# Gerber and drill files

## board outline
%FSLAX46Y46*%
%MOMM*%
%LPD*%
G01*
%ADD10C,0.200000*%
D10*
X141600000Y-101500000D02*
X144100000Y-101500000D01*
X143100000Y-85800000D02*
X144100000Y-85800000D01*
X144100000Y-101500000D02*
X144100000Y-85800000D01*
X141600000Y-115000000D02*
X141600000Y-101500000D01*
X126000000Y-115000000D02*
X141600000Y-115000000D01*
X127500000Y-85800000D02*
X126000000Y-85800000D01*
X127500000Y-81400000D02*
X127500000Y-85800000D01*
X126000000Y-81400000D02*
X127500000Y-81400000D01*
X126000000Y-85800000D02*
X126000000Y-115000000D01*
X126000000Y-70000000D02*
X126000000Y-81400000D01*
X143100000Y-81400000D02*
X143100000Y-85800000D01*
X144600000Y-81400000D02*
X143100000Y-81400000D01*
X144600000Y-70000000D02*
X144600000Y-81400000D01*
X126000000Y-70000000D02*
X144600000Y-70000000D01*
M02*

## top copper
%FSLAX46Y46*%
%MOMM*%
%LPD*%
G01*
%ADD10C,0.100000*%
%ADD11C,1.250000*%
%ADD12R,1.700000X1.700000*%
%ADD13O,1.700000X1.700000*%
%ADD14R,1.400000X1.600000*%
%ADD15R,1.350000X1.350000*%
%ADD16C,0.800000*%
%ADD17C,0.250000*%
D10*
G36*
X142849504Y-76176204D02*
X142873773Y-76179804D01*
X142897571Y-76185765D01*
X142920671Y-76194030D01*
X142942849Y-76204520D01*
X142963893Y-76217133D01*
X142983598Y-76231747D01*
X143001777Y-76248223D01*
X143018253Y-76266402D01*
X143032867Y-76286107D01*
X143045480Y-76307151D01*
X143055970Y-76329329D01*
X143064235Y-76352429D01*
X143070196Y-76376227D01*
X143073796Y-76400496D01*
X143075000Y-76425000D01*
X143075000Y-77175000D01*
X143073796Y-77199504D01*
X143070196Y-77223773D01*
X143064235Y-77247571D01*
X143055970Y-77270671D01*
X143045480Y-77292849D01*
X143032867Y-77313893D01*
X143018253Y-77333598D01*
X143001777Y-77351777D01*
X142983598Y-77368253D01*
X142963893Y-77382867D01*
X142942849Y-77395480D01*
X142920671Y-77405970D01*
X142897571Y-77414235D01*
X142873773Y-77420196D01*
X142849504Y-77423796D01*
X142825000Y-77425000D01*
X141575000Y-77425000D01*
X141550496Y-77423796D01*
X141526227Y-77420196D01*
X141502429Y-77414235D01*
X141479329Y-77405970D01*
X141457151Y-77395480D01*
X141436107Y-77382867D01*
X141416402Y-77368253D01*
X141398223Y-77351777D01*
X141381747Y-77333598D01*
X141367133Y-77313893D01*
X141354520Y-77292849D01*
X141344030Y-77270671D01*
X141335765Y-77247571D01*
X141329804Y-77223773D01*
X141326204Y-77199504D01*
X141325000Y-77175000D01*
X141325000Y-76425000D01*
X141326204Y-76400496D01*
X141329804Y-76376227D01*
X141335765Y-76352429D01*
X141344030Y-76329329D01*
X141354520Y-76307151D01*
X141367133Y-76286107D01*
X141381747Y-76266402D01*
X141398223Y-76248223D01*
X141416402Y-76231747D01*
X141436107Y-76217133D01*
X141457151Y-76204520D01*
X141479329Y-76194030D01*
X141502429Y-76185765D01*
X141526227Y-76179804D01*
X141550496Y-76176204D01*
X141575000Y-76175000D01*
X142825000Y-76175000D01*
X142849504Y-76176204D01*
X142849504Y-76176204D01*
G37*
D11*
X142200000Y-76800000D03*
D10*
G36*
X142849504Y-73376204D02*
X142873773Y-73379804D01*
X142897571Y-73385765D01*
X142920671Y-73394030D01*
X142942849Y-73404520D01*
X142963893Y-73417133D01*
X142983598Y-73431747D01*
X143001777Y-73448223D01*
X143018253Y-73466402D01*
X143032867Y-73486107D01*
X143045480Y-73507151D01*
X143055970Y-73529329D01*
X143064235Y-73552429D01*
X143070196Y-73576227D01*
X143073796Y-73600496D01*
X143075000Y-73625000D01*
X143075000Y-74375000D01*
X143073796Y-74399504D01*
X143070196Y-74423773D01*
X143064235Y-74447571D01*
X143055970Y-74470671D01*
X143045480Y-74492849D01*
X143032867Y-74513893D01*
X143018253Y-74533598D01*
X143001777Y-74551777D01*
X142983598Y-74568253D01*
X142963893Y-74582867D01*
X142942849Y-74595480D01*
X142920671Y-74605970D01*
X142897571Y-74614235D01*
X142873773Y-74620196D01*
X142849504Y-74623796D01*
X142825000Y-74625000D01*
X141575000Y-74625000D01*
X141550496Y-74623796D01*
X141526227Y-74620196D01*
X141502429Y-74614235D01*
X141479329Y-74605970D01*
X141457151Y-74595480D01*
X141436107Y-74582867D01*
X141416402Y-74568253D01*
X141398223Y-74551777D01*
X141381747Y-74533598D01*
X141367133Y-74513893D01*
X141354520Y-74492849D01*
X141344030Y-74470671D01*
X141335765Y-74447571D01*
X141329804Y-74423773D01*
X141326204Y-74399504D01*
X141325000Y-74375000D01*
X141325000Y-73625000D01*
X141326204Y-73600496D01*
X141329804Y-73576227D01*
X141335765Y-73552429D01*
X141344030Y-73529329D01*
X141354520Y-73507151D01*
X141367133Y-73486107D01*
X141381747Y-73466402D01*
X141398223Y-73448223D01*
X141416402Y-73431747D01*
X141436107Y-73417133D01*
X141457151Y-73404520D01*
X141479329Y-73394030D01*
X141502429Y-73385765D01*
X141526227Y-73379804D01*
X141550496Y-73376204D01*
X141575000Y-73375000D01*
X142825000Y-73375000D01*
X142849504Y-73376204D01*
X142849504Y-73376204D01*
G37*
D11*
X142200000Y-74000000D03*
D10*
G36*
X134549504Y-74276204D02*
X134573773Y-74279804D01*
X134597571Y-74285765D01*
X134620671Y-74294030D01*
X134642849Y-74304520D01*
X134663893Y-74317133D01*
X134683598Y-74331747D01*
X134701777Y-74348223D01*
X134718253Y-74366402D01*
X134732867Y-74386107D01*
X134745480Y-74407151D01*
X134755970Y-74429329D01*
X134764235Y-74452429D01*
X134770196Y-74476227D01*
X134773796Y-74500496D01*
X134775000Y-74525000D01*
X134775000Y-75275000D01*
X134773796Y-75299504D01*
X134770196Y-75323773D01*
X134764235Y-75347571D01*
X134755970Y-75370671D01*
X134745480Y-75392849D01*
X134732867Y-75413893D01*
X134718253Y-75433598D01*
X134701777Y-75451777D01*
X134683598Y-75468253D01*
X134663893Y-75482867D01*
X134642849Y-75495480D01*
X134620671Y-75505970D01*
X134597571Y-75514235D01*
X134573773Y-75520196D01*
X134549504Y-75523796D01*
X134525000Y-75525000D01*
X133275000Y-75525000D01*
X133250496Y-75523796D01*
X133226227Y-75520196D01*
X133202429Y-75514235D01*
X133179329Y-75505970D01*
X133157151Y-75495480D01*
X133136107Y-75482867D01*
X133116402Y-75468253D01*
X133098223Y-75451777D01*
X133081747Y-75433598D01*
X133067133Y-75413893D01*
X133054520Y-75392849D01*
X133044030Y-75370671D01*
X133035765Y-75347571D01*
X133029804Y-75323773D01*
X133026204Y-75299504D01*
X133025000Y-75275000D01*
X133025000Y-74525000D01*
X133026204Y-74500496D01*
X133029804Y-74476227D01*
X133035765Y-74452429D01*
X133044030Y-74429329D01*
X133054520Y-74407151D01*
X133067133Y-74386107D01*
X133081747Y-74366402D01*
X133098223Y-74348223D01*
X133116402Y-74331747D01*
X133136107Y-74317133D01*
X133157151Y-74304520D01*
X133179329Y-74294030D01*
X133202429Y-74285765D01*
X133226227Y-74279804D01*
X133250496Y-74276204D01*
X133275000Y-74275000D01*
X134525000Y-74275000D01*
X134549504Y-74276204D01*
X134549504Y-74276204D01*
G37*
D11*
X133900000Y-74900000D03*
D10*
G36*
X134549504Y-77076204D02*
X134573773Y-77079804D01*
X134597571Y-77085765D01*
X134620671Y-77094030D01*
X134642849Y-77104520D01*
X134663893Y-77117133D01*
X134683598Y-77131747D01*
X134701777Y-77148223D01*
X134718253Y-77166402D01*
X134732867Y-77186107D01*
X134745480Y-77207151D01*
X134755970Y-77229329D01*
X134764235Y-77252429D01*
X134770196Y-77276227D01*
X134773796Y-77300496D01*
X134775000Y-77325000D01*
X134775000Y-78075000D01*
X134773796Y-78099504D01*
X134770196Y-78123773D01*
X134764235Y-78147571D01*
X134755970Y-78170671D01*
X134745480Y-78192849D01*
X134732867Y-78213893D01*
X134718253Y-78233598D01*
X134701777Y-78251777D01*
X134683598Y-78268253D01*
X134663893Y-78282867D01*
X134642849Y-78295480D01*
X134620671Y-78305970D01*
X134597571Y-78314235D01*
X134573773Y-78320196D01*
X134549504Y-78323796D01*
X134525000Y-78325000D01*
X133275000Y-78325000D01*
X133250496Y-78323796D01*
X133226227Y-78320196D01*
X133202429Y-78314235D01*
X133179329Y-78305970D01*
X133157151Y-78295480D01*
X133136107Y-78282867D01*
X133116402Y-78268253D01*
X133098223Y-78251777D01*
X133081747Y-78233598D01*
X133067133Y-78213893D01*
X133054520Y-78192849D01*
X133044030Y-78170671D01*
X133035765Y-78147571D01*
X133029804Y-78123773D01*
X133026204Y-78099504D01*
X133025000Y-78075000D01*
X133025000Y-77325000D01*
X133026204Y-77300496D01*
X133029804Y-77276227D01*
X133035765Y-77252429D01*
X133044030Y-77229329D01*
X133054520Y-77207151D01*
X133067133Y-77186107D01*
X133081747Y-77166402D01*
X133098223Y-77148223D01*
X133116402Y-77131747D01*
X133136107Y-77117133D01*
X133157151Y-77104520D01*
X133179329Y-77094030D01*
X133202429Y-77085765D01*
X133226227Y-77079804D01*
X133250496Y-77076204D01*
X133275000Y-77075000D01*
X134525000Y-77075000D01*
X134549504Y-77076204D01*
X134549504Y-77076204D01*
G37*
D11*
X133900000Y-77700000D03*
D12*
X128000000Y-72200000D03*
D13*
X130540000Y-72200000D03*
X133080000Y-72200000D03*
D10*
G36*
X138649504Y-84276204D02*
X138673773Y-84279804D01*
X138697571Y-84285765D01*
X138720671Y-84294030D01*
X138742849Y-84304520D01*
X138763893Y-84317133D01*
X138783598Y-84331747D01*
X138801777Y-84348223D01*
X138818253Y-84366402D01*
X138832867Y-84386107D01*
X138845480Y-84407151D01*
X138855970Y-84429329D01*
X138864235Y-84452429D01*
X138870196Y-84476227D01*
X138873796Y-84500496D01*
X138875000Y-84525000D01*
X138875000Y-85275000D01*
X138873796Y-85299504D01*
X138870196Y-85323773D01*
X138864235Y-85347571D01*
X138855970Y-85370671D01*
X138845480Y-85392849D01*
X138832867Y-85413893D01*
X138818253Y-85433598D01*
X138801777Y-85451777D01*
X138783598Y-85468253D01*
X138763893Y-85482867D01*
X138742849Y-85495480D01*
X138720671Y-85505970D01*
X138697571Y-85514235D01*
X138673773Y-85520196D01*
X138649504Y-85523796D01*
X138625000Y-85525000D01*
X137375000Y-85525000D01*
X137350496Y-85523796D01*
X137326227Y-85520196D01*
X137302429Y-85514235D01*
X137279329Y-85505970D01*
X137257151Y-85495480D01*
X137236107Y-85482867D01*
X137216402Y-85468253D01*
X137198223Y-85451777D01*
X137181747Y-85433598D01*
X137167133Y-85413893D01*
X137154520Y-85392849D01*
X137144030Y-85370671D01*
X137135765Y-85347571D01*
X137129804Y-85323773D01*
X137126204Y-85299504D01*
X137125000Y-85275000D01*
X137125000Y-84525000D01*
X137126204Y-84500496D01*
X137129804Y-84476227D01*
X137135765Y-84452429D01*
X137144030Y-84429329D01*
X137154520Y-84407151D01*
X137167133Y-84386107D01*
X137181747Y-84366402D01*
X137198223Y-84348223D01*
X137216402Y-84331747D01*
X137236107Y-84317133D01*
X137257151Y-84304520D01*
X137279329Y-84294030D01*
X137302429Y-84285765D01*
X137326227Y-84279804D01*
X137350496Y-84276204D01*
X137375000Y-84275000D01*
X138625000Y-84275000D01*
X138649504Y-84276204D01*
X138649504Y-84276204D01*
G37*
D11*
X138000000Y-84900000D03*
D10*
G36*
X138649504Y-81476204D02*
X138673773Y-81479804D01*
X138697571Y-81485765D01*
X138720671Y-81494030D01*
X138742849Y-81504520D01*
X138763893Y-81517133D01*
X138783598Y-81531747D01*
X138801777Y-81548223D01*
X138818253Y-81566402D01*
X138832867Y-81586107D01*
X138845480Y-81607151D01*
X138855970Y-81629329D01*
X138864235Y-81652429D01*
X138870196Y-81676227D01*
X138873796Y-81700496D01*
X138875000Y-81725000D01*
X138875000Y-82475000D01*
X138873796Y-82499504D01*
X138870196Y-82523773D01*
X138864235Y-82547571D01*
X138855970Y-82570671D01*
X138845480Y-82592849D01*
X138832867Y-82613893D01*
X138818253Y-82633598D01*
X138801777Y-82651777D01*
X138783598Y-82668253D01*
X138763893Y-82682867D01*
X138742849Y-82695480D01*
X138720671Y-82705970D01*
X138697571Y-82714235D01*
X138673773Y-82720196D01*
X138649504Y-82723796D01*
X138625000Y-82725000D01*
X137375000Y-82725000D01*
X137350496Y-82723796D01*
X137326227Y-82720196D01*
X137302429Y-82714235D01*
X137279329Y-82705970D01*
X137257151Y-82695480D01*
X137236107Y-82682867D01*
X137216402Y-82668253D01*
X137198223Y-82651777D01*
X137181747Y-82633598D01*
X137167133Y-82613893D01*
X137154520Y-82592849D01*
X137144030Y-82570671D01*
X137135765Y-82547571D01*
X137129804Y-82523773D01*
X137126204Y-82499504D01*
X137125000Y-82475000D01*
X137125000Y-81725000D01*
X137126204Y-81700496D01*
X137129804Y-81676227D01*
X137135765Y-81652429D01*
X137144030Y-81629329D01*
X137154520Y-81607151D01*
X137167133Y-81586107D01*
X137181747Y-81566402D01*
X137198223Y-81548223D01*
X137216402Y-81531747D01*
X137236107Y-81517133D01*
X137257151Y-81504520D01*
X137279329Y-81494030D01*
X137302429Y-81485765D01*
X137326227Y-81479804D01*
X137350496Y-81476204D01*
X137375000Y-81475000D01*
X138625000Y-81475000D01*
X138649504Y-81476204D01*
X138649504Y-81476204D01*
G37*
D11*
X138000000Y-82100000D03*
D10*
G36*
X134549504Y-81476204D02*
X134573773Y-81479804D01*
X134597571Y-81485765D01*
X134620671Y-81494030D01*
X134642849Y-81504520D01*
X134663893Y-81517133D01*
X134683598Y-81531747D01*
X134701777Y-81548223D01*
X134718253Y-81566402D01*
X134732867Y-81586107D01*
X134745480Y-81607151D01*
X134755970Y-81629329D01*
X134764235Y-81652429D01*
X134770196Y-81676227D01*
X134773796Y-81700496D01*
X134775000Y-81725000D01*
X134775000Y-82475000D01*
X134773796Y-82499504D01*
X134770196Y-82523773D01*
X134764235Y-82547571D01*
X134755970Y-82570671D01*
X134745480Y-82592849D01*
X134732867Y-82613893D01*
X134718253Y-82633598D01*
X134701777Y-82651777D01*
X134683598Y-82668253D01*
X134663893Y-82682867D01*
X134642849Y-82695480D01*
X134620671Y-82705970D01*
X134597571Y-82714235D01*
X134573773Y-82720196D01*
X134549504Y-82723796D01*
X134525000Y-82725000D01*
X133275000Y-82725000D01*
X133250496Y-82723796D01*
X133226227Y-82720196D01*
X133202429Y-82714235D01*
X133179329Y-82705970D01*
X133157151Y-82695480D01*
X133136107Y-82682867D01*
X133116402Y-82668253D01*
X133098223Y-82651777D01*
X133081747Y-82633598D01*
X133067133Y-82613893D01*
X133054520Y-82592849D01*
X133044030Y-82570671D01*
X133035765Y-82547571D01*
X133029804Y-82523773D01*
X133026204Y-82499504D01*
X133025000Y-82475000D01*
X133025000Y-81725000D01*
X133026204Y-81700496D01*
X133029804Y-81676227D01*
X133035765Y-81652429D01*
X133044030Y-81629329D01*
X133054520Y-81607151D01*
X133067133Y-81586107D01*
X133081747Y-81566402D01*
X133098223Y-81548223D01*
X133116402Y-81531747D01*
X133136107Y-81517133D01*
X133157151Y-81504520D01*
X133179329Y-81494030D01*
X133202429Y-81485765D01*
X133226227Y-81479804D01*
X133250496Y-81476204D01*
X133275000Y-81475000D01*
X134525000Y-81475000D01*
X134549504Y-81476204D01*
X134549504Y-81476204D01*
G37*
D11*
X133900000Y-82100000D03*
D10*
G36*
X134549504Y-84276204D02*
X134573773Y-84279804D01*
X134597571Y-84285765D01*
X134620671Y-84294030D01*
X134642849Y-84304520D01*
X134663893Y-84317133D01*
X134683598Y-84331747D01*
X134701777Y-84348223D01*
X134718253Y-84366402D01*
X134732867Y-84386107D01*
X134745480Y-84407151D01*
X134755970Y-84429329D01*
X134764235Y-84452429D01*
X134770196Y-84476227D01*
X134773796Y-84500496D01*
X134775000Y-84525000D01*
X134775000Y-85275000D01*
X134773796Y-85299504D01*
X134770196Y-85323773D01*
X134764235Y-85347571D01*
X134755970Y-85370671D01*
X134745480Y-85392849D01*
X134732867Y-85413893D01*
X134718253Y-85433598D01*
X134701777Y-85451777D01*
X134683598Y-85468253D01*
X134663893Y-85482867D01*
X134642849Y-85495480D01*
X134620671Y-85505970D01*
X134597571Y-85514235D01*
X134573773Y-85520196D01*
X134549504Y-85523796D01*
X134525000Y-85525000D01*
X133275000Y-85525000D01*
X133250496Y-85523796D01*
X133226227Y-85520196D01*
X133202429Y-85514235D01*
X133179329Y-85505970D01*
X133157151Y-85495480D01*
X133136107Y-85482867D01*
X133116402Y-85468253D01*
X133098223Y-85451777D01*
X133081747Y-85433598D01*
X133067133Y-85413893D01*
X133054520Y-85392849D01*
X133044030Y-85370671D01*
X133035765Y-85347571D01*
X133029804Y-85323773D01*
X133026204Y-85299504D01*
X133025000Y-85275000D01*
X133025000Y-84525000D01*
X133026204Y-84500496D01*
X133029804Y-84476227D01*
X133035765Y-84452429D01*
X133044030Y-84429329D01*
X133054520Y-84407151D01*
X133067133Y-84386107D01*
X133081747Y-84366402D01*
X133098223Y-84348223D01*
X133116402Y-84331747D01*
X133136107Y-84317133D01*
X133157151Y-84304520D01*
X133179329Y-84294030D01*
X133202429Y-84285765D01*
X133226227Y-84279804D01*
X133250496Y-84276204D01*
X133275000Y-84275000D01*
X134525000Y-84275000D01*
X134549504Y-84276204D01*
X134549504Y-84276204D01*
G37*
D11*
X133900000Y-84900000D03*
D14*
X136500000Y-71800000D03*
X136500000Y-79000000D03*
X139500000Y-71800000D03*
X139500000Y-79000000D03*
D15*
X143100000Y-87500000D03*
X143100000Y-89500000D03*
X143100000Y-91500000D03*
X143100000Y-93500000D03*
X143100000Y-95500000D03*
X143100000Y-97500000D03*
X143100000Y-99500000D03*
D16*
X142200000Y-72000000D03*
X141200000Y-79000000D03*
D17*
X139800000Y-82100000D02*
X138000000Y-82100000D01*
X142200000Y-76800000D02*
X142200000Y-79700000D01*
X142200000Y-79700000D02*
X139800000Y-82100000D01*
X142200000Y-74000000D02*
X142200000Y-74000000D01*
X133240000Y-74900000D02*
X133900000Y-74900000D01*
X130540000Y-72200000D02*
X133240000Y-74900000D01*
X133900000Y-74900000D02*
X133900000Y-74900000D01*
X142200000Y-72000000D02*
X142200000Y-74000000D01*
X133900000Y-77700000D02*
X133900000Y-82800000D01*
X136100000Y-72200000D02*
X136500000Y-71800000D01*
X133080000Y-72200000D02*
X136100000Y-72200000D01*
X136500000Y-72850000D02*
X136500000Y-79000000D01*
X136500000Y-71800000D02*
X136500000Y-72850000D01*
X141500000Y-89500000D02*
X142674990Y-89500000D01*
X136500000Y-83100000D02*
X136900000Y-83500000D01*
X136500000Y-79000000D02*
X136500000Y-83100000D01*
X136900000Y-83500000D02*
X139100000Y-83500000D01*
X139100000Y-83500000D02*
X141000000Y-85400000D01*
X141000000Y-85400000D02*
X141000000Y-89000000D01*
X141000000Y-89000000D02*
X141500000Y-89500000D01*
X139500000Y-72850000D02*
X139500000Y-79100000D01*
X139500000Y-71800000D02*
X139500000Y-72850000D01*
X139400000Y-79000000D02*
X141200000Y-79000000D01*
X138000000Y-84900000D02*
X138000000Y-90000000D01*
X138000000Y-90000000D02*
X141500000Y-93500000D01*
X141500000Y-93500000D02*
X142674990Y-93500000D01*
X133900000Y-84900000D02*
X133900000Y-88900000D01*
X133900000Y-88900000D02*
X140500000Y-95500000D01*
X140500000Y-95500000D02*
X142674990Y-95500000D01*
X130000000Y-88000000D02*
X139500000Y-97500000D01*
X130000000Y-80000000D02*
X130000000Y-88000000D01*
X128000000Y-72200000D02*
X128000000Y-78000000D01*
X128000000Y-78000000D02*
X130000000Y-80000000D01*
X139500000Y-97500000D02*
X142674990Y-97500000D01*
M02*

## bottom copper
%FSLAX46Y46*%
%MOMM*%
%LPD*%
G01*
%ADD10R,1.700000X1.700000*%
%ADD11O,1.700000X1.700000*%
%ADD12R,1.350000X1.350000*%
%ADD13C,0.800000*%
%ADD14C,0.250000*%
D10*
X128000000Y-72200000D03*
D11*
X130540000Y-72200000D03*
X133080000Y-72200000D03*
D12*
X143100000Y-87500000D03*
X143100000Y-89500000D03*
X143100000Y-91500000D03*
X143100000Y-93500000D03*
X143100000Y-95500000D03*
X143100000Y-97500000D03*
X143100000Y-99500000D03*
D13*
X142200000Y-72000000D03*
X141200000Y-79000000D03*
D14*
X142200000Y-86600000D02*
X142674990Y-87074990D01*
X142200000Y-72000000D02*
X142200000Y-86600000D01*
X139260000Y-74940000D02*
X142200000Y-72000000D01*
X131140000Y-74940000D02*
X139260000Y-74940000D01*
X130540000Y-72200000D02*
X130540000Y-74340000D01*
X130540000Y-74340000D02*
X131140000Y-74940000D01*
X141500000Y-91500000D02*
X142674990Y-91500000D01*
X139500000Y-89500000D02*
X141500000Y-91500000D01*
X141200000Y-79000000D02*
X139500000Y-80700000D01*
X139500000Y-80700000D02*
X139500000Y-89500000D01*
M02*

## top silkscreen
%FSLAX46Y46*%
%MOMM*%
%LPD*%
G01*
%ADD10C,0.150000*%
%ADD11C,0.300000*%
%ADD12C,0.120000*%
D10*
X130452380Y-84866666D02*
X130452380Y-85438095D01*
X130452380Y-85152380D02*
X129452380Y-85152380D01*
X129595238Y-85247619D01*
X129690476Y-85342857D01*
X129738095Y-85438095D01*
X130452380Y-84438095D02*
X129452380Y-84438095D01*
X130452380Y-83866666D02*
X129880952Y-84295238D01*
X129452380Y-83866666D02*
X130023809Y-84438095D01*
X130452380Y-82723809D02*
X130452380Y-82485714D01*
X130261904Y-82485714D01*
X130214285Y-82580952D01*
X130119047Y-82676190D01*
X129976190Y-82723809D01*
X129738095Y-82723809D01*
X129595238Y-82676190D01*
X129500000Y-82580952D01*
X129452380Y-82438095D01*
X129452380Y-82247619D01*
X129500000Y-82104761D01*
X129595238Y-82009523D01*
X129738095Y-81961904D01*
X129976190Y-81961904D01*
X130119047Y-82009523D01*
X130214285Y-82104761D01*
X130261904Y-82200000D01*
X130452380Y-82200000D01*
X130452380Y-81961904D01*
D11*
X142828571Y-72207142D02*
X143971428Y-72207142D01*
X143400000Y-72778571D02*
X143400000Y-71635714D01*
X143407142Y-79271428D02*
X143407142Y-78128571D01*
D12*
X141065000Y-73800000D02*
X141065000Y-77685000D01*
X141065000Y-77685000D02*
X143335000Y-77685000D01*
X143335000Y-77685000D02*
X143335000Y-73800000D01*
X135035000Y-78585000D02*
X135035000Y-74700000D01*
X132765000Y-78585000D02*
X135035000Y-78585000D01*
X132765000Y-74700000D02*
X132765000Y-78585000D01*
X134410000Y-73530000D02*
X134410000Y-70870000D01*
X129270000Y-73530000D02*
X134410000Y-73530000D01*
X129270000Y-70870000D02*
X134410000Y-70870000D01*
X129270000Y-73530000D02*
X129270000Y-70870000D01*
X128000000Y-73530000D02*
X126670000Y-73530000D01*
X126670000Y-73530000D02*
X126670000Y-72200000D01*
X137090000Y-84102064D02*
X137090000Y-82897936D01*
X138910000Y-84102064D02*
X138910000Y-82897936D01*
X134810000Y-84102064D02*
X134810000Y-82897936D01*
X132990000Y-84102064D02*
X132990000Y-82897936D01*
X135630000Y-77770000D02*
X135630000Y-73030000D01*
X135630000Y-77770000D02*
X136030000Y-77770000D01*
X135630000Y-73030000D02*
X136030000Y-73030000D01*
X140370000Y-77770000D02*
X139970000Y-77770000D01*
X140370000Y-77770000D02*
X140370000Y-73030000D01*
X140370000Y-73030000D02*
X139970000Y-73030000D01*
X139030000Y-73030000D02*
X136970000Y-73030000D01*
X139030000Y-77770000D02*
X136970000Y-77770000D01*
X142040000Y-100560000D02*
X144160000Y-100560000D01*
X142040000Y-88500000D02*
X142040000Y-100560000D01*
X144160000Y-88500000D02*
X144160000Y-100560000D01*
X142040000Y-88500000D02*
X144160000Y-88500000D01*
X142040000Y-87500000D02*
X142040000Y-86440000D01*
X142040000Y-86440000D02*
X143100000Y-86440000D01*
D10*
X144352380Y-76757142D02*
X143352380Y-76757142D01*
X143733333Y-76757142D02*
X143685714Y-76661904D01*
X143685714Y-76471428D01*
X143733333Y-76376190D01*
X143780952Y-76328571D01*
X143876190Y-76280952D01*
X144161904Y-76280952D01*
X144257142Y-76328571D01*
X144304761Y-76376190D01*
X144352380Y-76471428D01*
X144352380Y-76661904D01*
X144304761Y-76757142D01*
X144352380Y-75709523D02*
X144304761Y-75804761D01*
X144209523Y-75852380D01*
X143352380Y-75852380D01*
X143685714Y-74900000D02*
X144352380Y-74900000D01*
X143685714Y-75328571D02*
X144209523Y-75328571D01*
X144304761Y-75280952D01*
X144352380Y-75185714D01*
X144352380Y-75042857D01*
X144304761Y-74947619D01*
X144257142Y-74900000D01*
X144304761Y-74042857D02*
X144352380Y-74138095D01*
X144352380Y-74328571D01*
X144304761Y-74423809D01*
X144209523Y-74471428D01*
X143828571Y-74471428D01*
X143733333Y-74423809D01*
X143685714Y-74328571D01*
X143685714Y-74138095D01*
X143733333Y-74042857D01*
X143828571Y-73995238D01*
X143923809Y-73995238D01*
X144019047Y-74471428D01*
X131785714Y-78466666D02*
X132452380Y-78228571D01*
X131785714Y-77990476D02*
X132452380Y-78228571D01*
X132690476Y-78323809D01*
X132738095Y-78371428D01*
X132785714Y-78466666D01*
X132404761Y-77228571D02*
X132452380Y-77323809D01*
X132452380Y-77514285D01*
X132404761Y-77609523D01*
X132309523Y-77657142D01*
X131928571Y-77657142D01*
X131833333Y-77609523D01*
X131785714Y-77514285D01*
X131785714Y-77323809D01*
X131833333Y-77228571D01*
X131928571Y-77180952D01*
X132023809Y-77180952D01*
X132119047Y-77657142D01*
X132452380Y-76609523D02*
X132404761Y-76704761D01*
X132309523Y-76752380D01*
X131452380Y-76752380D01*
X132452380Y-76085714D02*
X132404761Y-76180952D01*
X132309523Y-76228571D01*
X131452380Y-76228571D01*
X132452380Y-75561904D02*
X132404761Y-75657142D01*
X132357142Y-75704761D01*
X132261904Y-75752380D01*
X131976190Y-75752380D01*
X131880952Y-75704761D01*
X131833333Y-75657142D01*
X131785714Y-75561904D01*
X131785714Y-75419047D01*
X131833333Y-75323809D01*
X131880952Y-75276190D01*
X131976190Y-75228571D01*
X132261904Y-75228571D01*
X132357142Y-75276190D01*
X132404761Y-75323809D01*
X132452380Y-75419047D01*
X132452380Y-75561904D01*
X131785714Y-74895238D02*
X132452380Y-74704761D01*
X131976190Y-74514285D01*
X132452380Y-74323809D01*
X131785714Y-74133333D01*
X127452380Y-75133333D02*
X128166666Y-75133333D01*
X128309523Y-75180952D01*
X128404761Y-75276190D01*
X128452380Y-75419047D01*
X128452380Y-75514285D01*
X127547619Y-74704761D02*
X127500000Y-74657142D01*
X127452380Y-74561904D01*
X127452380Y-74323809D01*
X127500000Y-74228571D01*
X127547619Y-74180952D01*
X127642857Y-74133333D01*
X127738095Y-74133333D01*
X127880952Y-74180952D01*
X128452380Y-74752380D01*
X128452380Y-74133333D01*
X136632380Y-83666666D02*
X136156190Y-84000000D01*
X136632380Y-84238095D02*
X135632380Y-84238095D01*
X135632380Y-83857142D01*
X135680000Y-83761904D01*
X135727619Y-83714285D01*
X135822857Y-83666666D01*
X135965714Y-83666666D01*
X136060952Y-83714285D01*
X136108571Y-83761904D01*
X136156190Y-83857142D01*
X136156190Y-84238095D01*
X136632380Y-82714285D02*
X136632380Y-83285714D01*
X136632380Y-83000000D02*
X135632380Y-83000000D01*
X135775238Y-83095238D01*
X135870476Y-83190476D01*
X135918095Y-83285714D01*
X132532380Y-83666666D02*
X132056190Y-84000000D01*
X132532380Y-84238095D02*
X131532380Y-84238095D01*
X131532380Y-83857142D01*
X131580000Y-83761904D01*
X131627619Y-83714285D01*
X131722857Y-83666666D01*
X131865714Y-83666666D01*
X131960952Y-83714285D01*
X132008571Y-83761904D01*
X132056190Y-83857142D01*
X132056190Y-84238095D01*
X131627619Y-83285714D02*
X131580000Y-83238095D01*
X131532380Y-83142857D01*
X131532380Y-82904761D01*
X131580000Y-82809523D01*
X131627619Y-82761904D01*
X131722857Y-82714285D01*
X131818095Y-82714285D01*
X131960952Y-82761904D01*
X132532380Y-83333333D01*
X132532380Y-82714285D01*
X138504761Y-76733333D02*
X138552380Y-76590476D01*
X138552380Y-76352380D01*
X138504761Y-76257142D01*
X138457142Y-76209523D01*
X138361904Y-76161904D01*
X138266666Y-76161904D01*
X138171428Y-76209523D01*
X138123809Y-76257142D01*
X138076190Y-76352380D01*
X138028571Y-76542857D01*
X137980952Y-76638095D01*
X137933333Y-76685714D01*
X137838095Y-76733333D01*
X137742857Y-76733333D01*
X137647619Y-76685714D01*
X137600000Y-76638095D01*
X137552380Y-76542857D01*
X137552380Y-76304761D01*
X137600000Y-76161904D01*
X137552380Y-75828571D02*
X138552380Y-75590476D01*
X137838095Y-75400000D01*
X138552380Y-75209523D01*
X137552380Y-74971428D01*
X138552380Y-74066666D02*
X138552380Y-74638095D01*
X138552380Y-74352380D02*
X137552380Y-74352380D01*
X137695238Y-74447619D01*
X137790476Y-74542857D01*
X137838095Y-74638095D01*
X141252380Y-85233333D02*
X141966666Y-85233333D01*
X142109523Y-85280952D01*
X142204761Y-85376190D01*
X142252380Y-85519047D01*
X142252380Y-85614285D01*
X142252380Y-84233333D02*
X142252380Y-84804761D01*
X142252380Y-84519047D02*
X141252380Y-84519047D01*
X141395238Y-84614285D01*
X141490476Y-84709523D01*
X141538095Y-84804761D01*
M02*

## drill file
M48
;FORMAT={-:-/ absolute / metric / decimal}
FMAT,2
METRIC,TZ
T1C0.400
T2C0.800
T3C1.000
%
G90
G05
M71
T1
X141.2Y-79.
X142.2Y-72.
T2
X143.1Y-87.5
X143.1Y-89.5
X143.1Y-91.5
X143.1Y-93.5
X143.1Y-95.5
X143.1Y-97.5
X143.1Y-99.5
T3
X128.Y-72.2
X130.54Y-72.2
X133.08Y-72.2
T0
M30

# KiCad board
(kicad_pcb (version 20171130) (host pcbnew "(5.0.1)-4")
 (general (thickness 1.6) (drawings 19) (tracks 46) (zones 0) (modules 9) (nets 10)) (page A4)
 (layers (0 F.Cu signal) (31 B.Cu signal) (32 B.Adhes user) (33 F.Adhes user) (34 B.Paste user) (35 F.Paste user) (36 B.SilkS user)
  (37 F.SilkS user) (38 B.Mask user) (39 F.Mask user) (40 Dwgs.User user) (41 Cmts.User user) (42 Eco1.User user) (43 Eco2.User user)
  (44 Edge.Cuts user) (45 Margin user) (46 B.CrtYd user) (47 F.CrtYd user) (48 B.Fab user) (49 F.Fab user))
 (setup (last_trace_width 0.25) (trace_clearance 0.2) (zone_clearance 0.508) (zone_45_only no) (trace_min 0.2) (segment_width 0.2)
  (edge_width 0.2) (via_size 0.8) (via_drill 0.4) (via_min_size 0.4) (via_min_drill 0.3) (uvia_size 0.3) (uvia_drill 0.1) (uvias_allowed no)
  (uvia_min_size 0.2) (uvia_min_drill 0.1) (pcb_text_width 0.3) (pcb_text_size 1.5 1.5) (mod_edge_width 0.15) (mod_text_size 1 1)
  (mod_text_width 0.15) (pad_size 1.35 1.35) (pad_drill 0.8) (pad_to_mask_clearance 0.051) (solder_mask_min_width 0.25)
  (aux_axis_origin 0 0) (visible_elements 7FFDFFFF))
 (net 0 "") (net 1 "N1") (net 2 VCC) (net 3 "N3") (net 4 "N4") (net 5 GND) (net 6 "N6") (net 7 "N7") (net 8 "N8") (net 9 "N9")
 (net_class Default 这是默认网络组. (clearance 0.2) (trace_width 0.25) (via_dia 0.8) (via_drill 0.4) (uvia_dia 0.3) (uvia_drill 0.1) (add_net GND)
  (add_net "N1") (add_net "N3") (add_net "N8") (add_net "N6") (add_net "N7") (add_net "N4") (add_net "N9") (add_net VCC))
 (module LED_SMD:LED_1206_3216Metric (layer F.Cu) (at 142.2 75.4 90)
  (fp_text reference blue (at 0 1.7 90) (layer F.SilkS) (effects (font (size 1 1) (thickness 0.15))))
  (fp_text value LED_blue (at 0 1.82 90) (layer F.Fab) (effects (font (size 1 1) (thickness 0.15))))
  (fp_line (start 1.6 -1.135) (end -2.285 -1.135) (layer F.SilkS) (width 0.12))
  (fp_line (start -2.285 -1.135) (end -2.285 1.135) (layer F.SilkS) (width 0.12))
  (fp_line (start -2.285 1.135) (end 1.6 1.135) (layer F.SilkS) (width 0.12))
  (pad 1 smd roundrect (at -1.4 0 90) (size 1.25 1.75) (layers F.Cu F.Paste F.Mask) (roundrect_rratio 0.2) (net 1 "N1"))
  (pad 2 smd roundrect (at 1.4 0 90) (size 1.25 1.75) (layers F.Cu F.Paste F.Mask) (roundrect_rratio 0.2) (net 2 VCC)))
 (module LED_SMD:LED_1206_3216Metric (layer F.Cu) (at 133.9 76.3 90)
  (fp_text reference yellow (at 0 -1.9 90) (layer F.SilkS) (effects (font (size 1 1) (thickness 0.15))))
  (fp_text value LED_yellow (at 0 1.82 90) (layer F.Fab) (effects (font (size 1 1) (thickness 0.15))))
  (fp_line (start -2.285 1.135) (end 1.6 1.135) (layer F.SilkS) (width 0.12))
  (fp_line (start -2.285 -1.135) (end -2.285 1.135) (layer F.SilkS) (width 0.12))
  (fp_line (start 1.6 -1.135) (end -2.285 -1.135) (layer F.SilkS) (width 0.12))
  (pad 2 smd roundrect (at 1.4 0 90) (size 1.25 1.75) (layers F.Cu F.Paste F.Mask) (roundrect_rratio 0.2) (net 2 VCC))
  (pad 1 smd roundrect (at -1.4 0 90) (size 1.25 1.75) (layers F.Cu F.Paste F.Mask) (roundrect_rratio 0.2) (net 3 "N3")))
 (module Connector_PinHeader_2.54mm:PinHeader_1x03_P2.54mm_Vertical (layer F.Cu) (at 128 72.2 90)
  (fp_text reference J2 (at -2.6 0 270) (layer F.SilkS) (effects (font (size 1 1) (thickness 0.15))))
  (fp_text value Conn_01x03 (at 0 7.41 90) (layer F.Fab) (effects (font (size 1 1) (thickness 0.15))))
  (fp_line (start -1.33 6.41) (end 1.33 6.41) (layer F.SilkS) (width 0.12))
  (fp_line (start -1.33 1.27) (end -1.33 6.41) (layer F.SilkS) (width 0.12))
  (fp_line (start 1.33 1.27) (end 1.33 6.41) (layer F.SilkS) (width 0.12))
  (fp_line (start -1.33 1.27) (end 1.33 1.27) (layer F.SilkS) (width 0.12))
  (fp_line (start -1.33 0) (end -1.33 -1.33) (layer F.SilkS) (width 0.12))
  (fp_line (start -1.33 -1.33) (end 0 -1.33) (layer F.SilkS) (width 0.12))
  (pad 1 thru_hole rect (at 0 0 90) (size 1.7 1.7) (drill 1) (layers *.Cu *.Mask) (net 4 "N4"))
  (pad 2 thru_hole oval (at 0 2.54 90) (size 1.7 1.7) (drill 1) (layers *.Cu *.Mask) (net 2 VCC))
  (pad 3 thru_hole oval (at 0 5.08 90) (size 1.7 1.7) (drill 1) (layers *.Cu *.Mask) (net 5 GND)))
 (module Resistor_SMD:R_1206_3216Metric (layer F.Cu) (at 138 83.5 90)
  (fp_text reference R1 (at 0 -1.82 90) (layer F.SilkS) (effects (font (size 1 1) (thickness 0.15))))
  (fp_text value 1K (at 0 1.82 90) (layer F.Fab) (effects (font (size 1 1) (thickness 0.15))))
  (fp_line (start -0.602064 -0.91) (end 0.602064 -0.91) (layer F.SilkS) (width 0.12))
  (fp_line (start -0.602064 0.91) (end 0.602064 0.91) (layer F.SilkS) (width 0.12))
  (pad 1 smd roundrect (at -1.4 0 90) (size 1.25 1.75) (layers F.Cu F.Paste F.Mask) (roundrect_rratio 0.2) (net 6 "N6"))
  (pad 2 smd roundrect (at 1.4 0 90) (size 1.25 1.75) (layers F.Cu F.Paste F.Mask) (roundrect_rratio 0.2) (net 1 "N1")))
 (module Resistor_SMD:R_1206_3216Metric (layer F.Cu) (at 133.9 83.5 90)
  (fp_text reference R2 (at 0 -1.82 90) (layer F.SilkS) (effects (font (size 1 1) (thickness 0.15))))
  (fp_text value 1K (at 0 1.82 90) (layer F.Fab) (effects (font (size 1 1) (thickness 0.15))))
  (fp_line (start -0.602064 0.91) (end 0.602064 0.91) (layer F.SilkS) (width 0.12))
  (fp_line (start -0.602064 -0.91) (end 0.602064 -0.91) (layer F.SilkS) (width 0.12))
  (pad 2 smd roundrect (at 1.4 0 90) (size 1.25 1.75) (layers F.Cu F.Paste F.Mask) (roundrect_rratio 0.2) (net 3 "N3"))
  (pad 1 smd roundrect (at -1.4 0 90) (size 1.25 1.75) (layers F.Cu F.Paste F.Mask) (roundrect_rratio 0.2) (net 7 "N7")))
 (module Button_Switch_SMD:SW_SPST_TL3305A (layer F.Cu) (at 138 75.4 90)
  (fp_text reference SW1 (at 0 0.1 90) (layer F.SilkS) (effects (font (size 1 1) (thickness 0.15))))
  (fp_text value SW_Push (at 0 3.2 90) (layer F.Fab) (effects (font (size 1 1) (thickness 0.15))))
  (fp_line (start -2.37 -2.37) (end 2.37 -2.37) (layer F.SilkS) (width 0.12))
  (fp_line (start -2.37 -2.37) (end -2.37 -1.97) (layer F.SilkS) (width 0.12))
  (fp_line (start 2.37 -2.37) (end 2.37 -1.97) (layer F.SilkS) (width 0.12))
  (fp_line (start -2.37 2.37) (end -2.37 1.97) (layer F.SilkS) (width 0.12))
  (fp_line (start -2.37 2.37) (end 2.37 2.37) (layer F.SilkS) (width 0.12))
  (fp_line (start 2.37 2.37) (end 2.37 1.97) (layer F.SilkS) (width 0.12))
  (fp_line (start 2.37 1.03) (end 2.37 -1.03) (layer F.SilkS) (width 0.12))
  (fp_line (start -2.37 1.03) (end -2.37 -1.03) (layer F.SilkS) (width 0.12))
  (pad 1 smd rect (at 3.6 -1.5 90) (size 1.6 1.4) (layers F.Cu F.Paste F.Mask) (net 5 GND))
  (pad 1 smd rect (at -3.6 -1.5 90) (size 1.6 1.4) (layers F.Cu F.Paste F.Mask) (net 5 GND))
  (pad 2 smd rect (at 3.6 1.5 90) (size 1.6 1.4) (layers F.Cu F.Paste F.Mask) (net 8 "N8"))
  (pad 2 smd rect (at -3.6 1.5 90) (size 1.6 1.4) (layers F.Cu F.Paste F.Mask) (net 8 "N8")))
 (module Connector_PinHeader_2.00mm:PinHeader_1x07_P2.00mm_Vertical (layer F.Cu) (at 143.1 87.5)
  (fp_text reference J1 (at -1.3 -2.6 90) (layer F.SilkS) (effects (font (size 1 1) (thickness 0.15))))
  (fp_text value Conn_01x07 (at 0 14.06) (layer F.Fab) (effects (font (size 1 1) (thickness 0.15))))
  (fp_line (start -1.06 13.06) (end 1.06 13.06) (layer F.SilkS) (width 0.12))
  (fp_line (start -1.06 1) (end -1.06 13.06) (layer F.SilkS) (width 0.12))
  (fp_line (start 1.06 1) (end 1.06 13.06) (layer F.SilkS) (width 0.12))
  (fp_line (start -1.06 1) (end 1.06 1) (layer F.SilkS) (width 0.12))
  (fp_line (start -1.06 0) (end -1.06 -1.06) (layer F.SilkS) (width 0.12))
  (fp_line (start -1.06 -1.06) (end 0 -1.06) (layer F.SilkS) (width 0.12))
  (pad 1 thru_hole rect (at 0 0) (size 1.35 1.35) (drill 0.8) (layers *.Cu *.Mask) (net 2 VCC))
  (pad 2 thru_hole rect (at 0 2) (size 1.35 1.35) (drill 0.8) (layers *.Cu *.Mask) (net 5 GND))
  (pad 3 thru_hole rect (at 0 4) (size 1.35 1.35) (drill 0.8) (layers *.Cu *.Mask) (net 8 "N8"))
  (pad 4 thru_hole rect (at 0 6) (size 1.35 1.35) (drill 0.8) (layers *.Cu *.Mask) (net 6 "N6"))
  (pad 5 thru_hole rect (at 0 8) (size 1.35 1.35) (drill 0.8) (layers *.Cu *.Mask) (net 7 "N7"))
  (pad 6 thru_hole rect (at 0 10) (size 1.35 1.35) (drill 0.8) (layers *.Cu *.Mask) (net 4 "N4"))
  (pad 7 thru_hole rect (at 0 12) (size 1.35 1.35) (drill 0.8) (layers *.Cu *.Mask) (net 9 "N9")))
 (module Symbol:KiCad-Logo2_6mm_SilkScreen (layer B.Cu) (at 134 110)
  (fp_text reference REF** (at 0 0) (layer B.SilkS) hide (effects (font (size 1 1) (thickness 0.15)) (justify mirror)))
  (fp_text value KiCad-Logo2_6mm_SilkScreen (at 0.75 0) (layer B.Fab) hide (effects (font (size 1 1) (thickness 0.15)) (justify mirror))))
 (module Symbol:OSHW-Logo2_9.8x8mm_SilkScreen (layer B.Cu) (at 134 100.8)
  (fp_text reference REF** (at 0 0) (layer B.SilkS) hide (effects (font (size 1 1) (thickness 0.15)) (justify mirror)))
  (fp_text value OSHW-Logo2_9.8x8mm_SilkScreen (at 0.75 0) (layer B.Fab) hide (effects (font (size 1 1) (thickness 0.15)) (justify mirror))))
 (gr_line (start 141.6 101.5) (end 144.1 101.5) (layer Edge.Cuts) (width 0.2))
 (gr_line (start 143.1 85.8) (end 144.1 85.8) (layer Edge.Cuts) (width 0.2))
 (gr_line (start 144.1 101.5) (end 144.1 85.8) (layer Edge.Cuts) (width 0.2))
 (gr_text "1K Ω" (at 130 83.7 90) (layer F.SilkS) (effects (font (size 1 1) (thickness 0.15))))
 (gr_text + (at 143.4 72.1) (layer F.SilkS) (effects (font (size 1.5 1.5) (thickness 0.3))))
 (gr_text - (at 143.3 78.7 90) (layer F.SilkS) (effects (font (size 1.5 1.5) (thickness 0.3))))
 (gr_line (start 141.6 115) (end 141.6 101.5) (layer Edge.Cuts) (width 0.2))
 (gr_line (start 126 115) (end 141.6 115) (layer Edge.Cuts) (width 0.2))
 (gr_line (start 127.5 85.8) (end 126 85.8) (layer Edge.Cuts) (width 0.2))
 (gr_line (start 127.5 81.4) (end 127.5 85.8) (layer Edge.Cuts) (width 0.2))
 (gr_line (start 126 81.4) (end 127.5 81.4) (layer Edge.Cuts) (width 0.2))
 (gr_line (start 126 85.8) (end 126 115) (layer Edge.Cuts) (width 0.2))
 (gr_line (start 126 70) (end 126 81.4) (layer Edge.Cuts) (width 0.2))
 (gr_line (start 143.1 81.4) (end 143.1 85.8) (layer Edge.Cuts) (width 0.2))
 (gr_line (start 144.6 81.4) (end 143.1 81.4) (layer Edge.Cuts) (width 0.2))
 (gr_line (start 144.6 70) (end 144.6 81.4) (layer Edge.Cuts) (width 0.2))
 (gr_line (start 126 70) (end 144.6 70) (layer Edge.Cuts) (width 0.2))
 (segment (start 139.8 82.1) (end 138 82.1) (width 0.25) (layer F.Cu) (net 1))
 (segment (start 142.2 76.8) (end 142.2 79.7) (width 0.25) (layer F.Cu) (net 1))
 (segment (start 142.2 79.7) (end 139.8 82.1) (width 0.25) (layer F.Cu) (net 1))
 (segment (start 142.2 74) (end 142.2 74) (width 0.25) (layer F.Cu) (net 2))
 (segment (start 133.24 74.9) (end 133.9 74.9) (width 0.25) (layer F.Cu) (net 2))
 (segment (start 130.54 72.2) (end 133.24 74.9) (width 0.25) (layer F.Cu) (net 2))
 (segment (start 133.9 74.9) (end 133.9 74.9) (width 0.25) (layer F.Cu) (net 2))
 (via (at 142.2 72) (size 0.8) (drill 0.4) (layers F.Cu B.Cu) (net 2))
 (segment (start 142.2 72) (end 142.2 74) (width 0.25) (layer F.Cu) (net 2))
 (segment (start 142.2 86.6) (end 142.67499 87.07499) (width 0.25) (layer B.Cu) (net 2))
 (segment (start 142.2 72) (end 142.2 86.6) (width 0.25) (layer B.Cu) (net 2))
 (segment (start 139.26 74.94) (end 142.2 72) (width 0.25) (layer B.Cu) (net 2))
 (segment (start 131.14 74.94) (end 139.26 74.94) (width 0.25) (layer B.Cu) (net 2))
 (segment (start 130.54 72.2) (end 130.54 74.34) (width 0.25) (layer B.Cu) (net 2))
 (segment (start 130.54 74.34) (end 131.14 74.94) (width 0.25) (layer B.Cu) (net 2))
 (segment (start 133.9 77.7) (end 133.9 82.8) (width 0.25) (layer F.Cu) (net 3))
 (segment (start 136.1 72.2) (end 136.5 71.8) (width 0.25) (layer F.Cu) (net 5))
 (segment (start 133.08 72.2) (end 136.1 72.2) (width 0.25) (layer F.Cu) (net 5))
 (segment (start 136.5 72.85) (end 136.5 79) (width 0.25) (layer F.Cu) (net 5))
 (segment (start 136.5 71.8) (end 136.5 72.85) (width 0.25) (layer F.Cu) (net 5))
 (segment (start 141.5 89.5) (end 142.67499 89.5) (width 0.25) (layer F.Cu) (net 5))
 (segment (start 136.5 83.1) (end 136.9 83.5) (width 0.25) (layer F.Cu) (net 5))
 (segment (start 136.5 79) (end 136.5 83.1) (width 0.25) (layer F.Cu) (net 5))
 (segment (start 136.9 83.5) (end 139.1 83.5) (width 0.25) (layer F.Cu) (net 5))
 (segment (start 139.1 83.5) (end 141 85.4) (width 0.25) (layer F.Cu) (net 5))
 (segment (start 141 85.4) (end 141 89) (width 0.25) (layer F.Cu) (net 5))
 (segment (start 141 89) (end 141.5 89.5) (width 0.25) (layer F.Cu) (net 5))
 (via (at 141.2 79) (size 0.8) (drill 0.4) (layers F.Cu B.Cu) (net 8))
 (segment (start 139.5 72.85) (end 139.5 79.1) (width 0.25) (layer F.Cu) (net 8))
 (segment (start 139.5 71.8) (end 139.5 72.85) (width 0.25) (layer F.Cu) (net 8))
 (segment (start 139.4 79) (end 141.2 79) (width 0.25) (layer F.Cu) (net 8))
 (segment (start 141.5 91.5) (end 142.67499 91.5) (width 0.25) (layer B.Cu) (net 8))
 (segment (start 139.5 89.5) (end 141.5 91.5) (width 0.25) (layer B.Cu) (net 8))
 (segment (start 141.2 79) (end 139.5 80.7) (width 0.25) (layer B.Cu) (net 8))
 (segment (start 139.5 80.7) (end 139.5 89.5) (width 0.25) (layer B.Cu) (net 8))
 (segment (start 138 84.9) (end 138 90) (width 0.25) (layer F.Cu) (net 6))
 (segment (start 138 90) (end 141.5 93.5) (width 0.25) (layer F.Cu) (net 6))
 (segment (start 141.5 93.5) (end 142.67499 93.5) (width 0.25) (layer F.Cu) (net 6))
 (segment (start 133.9 84.9) (end 133.9 88.9) (width 0.25) (layer F.Cu) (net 7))
 (segment (start 133.9 88.9) (end 140.5 95.5) (width 0.25) (layer F.Cu) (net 7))
 (segment (start 140.5 95.5) (end 142.67499 95.5) (width 0.25) (layer F.Cu) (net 7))
 (segment (start 130 88) (end 139.5 97.5) (width 0.25) (layer F.Cu) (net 4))
 (segment (start 130 80) (end 130 88) (width 0.25) (layer F.Cu) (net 4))
 (segment (start 128 72.2) (end 128 78) (width 0.25) (layer F.Cu) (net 4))
 (segment (start 128 78) (end 130 80) (width 0.25) (layer F.Cu) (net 4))
 (segment (start 139.5 97.5) (end 142.67499 97.5) (width 0.25) (layer F.Cu) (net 4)))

